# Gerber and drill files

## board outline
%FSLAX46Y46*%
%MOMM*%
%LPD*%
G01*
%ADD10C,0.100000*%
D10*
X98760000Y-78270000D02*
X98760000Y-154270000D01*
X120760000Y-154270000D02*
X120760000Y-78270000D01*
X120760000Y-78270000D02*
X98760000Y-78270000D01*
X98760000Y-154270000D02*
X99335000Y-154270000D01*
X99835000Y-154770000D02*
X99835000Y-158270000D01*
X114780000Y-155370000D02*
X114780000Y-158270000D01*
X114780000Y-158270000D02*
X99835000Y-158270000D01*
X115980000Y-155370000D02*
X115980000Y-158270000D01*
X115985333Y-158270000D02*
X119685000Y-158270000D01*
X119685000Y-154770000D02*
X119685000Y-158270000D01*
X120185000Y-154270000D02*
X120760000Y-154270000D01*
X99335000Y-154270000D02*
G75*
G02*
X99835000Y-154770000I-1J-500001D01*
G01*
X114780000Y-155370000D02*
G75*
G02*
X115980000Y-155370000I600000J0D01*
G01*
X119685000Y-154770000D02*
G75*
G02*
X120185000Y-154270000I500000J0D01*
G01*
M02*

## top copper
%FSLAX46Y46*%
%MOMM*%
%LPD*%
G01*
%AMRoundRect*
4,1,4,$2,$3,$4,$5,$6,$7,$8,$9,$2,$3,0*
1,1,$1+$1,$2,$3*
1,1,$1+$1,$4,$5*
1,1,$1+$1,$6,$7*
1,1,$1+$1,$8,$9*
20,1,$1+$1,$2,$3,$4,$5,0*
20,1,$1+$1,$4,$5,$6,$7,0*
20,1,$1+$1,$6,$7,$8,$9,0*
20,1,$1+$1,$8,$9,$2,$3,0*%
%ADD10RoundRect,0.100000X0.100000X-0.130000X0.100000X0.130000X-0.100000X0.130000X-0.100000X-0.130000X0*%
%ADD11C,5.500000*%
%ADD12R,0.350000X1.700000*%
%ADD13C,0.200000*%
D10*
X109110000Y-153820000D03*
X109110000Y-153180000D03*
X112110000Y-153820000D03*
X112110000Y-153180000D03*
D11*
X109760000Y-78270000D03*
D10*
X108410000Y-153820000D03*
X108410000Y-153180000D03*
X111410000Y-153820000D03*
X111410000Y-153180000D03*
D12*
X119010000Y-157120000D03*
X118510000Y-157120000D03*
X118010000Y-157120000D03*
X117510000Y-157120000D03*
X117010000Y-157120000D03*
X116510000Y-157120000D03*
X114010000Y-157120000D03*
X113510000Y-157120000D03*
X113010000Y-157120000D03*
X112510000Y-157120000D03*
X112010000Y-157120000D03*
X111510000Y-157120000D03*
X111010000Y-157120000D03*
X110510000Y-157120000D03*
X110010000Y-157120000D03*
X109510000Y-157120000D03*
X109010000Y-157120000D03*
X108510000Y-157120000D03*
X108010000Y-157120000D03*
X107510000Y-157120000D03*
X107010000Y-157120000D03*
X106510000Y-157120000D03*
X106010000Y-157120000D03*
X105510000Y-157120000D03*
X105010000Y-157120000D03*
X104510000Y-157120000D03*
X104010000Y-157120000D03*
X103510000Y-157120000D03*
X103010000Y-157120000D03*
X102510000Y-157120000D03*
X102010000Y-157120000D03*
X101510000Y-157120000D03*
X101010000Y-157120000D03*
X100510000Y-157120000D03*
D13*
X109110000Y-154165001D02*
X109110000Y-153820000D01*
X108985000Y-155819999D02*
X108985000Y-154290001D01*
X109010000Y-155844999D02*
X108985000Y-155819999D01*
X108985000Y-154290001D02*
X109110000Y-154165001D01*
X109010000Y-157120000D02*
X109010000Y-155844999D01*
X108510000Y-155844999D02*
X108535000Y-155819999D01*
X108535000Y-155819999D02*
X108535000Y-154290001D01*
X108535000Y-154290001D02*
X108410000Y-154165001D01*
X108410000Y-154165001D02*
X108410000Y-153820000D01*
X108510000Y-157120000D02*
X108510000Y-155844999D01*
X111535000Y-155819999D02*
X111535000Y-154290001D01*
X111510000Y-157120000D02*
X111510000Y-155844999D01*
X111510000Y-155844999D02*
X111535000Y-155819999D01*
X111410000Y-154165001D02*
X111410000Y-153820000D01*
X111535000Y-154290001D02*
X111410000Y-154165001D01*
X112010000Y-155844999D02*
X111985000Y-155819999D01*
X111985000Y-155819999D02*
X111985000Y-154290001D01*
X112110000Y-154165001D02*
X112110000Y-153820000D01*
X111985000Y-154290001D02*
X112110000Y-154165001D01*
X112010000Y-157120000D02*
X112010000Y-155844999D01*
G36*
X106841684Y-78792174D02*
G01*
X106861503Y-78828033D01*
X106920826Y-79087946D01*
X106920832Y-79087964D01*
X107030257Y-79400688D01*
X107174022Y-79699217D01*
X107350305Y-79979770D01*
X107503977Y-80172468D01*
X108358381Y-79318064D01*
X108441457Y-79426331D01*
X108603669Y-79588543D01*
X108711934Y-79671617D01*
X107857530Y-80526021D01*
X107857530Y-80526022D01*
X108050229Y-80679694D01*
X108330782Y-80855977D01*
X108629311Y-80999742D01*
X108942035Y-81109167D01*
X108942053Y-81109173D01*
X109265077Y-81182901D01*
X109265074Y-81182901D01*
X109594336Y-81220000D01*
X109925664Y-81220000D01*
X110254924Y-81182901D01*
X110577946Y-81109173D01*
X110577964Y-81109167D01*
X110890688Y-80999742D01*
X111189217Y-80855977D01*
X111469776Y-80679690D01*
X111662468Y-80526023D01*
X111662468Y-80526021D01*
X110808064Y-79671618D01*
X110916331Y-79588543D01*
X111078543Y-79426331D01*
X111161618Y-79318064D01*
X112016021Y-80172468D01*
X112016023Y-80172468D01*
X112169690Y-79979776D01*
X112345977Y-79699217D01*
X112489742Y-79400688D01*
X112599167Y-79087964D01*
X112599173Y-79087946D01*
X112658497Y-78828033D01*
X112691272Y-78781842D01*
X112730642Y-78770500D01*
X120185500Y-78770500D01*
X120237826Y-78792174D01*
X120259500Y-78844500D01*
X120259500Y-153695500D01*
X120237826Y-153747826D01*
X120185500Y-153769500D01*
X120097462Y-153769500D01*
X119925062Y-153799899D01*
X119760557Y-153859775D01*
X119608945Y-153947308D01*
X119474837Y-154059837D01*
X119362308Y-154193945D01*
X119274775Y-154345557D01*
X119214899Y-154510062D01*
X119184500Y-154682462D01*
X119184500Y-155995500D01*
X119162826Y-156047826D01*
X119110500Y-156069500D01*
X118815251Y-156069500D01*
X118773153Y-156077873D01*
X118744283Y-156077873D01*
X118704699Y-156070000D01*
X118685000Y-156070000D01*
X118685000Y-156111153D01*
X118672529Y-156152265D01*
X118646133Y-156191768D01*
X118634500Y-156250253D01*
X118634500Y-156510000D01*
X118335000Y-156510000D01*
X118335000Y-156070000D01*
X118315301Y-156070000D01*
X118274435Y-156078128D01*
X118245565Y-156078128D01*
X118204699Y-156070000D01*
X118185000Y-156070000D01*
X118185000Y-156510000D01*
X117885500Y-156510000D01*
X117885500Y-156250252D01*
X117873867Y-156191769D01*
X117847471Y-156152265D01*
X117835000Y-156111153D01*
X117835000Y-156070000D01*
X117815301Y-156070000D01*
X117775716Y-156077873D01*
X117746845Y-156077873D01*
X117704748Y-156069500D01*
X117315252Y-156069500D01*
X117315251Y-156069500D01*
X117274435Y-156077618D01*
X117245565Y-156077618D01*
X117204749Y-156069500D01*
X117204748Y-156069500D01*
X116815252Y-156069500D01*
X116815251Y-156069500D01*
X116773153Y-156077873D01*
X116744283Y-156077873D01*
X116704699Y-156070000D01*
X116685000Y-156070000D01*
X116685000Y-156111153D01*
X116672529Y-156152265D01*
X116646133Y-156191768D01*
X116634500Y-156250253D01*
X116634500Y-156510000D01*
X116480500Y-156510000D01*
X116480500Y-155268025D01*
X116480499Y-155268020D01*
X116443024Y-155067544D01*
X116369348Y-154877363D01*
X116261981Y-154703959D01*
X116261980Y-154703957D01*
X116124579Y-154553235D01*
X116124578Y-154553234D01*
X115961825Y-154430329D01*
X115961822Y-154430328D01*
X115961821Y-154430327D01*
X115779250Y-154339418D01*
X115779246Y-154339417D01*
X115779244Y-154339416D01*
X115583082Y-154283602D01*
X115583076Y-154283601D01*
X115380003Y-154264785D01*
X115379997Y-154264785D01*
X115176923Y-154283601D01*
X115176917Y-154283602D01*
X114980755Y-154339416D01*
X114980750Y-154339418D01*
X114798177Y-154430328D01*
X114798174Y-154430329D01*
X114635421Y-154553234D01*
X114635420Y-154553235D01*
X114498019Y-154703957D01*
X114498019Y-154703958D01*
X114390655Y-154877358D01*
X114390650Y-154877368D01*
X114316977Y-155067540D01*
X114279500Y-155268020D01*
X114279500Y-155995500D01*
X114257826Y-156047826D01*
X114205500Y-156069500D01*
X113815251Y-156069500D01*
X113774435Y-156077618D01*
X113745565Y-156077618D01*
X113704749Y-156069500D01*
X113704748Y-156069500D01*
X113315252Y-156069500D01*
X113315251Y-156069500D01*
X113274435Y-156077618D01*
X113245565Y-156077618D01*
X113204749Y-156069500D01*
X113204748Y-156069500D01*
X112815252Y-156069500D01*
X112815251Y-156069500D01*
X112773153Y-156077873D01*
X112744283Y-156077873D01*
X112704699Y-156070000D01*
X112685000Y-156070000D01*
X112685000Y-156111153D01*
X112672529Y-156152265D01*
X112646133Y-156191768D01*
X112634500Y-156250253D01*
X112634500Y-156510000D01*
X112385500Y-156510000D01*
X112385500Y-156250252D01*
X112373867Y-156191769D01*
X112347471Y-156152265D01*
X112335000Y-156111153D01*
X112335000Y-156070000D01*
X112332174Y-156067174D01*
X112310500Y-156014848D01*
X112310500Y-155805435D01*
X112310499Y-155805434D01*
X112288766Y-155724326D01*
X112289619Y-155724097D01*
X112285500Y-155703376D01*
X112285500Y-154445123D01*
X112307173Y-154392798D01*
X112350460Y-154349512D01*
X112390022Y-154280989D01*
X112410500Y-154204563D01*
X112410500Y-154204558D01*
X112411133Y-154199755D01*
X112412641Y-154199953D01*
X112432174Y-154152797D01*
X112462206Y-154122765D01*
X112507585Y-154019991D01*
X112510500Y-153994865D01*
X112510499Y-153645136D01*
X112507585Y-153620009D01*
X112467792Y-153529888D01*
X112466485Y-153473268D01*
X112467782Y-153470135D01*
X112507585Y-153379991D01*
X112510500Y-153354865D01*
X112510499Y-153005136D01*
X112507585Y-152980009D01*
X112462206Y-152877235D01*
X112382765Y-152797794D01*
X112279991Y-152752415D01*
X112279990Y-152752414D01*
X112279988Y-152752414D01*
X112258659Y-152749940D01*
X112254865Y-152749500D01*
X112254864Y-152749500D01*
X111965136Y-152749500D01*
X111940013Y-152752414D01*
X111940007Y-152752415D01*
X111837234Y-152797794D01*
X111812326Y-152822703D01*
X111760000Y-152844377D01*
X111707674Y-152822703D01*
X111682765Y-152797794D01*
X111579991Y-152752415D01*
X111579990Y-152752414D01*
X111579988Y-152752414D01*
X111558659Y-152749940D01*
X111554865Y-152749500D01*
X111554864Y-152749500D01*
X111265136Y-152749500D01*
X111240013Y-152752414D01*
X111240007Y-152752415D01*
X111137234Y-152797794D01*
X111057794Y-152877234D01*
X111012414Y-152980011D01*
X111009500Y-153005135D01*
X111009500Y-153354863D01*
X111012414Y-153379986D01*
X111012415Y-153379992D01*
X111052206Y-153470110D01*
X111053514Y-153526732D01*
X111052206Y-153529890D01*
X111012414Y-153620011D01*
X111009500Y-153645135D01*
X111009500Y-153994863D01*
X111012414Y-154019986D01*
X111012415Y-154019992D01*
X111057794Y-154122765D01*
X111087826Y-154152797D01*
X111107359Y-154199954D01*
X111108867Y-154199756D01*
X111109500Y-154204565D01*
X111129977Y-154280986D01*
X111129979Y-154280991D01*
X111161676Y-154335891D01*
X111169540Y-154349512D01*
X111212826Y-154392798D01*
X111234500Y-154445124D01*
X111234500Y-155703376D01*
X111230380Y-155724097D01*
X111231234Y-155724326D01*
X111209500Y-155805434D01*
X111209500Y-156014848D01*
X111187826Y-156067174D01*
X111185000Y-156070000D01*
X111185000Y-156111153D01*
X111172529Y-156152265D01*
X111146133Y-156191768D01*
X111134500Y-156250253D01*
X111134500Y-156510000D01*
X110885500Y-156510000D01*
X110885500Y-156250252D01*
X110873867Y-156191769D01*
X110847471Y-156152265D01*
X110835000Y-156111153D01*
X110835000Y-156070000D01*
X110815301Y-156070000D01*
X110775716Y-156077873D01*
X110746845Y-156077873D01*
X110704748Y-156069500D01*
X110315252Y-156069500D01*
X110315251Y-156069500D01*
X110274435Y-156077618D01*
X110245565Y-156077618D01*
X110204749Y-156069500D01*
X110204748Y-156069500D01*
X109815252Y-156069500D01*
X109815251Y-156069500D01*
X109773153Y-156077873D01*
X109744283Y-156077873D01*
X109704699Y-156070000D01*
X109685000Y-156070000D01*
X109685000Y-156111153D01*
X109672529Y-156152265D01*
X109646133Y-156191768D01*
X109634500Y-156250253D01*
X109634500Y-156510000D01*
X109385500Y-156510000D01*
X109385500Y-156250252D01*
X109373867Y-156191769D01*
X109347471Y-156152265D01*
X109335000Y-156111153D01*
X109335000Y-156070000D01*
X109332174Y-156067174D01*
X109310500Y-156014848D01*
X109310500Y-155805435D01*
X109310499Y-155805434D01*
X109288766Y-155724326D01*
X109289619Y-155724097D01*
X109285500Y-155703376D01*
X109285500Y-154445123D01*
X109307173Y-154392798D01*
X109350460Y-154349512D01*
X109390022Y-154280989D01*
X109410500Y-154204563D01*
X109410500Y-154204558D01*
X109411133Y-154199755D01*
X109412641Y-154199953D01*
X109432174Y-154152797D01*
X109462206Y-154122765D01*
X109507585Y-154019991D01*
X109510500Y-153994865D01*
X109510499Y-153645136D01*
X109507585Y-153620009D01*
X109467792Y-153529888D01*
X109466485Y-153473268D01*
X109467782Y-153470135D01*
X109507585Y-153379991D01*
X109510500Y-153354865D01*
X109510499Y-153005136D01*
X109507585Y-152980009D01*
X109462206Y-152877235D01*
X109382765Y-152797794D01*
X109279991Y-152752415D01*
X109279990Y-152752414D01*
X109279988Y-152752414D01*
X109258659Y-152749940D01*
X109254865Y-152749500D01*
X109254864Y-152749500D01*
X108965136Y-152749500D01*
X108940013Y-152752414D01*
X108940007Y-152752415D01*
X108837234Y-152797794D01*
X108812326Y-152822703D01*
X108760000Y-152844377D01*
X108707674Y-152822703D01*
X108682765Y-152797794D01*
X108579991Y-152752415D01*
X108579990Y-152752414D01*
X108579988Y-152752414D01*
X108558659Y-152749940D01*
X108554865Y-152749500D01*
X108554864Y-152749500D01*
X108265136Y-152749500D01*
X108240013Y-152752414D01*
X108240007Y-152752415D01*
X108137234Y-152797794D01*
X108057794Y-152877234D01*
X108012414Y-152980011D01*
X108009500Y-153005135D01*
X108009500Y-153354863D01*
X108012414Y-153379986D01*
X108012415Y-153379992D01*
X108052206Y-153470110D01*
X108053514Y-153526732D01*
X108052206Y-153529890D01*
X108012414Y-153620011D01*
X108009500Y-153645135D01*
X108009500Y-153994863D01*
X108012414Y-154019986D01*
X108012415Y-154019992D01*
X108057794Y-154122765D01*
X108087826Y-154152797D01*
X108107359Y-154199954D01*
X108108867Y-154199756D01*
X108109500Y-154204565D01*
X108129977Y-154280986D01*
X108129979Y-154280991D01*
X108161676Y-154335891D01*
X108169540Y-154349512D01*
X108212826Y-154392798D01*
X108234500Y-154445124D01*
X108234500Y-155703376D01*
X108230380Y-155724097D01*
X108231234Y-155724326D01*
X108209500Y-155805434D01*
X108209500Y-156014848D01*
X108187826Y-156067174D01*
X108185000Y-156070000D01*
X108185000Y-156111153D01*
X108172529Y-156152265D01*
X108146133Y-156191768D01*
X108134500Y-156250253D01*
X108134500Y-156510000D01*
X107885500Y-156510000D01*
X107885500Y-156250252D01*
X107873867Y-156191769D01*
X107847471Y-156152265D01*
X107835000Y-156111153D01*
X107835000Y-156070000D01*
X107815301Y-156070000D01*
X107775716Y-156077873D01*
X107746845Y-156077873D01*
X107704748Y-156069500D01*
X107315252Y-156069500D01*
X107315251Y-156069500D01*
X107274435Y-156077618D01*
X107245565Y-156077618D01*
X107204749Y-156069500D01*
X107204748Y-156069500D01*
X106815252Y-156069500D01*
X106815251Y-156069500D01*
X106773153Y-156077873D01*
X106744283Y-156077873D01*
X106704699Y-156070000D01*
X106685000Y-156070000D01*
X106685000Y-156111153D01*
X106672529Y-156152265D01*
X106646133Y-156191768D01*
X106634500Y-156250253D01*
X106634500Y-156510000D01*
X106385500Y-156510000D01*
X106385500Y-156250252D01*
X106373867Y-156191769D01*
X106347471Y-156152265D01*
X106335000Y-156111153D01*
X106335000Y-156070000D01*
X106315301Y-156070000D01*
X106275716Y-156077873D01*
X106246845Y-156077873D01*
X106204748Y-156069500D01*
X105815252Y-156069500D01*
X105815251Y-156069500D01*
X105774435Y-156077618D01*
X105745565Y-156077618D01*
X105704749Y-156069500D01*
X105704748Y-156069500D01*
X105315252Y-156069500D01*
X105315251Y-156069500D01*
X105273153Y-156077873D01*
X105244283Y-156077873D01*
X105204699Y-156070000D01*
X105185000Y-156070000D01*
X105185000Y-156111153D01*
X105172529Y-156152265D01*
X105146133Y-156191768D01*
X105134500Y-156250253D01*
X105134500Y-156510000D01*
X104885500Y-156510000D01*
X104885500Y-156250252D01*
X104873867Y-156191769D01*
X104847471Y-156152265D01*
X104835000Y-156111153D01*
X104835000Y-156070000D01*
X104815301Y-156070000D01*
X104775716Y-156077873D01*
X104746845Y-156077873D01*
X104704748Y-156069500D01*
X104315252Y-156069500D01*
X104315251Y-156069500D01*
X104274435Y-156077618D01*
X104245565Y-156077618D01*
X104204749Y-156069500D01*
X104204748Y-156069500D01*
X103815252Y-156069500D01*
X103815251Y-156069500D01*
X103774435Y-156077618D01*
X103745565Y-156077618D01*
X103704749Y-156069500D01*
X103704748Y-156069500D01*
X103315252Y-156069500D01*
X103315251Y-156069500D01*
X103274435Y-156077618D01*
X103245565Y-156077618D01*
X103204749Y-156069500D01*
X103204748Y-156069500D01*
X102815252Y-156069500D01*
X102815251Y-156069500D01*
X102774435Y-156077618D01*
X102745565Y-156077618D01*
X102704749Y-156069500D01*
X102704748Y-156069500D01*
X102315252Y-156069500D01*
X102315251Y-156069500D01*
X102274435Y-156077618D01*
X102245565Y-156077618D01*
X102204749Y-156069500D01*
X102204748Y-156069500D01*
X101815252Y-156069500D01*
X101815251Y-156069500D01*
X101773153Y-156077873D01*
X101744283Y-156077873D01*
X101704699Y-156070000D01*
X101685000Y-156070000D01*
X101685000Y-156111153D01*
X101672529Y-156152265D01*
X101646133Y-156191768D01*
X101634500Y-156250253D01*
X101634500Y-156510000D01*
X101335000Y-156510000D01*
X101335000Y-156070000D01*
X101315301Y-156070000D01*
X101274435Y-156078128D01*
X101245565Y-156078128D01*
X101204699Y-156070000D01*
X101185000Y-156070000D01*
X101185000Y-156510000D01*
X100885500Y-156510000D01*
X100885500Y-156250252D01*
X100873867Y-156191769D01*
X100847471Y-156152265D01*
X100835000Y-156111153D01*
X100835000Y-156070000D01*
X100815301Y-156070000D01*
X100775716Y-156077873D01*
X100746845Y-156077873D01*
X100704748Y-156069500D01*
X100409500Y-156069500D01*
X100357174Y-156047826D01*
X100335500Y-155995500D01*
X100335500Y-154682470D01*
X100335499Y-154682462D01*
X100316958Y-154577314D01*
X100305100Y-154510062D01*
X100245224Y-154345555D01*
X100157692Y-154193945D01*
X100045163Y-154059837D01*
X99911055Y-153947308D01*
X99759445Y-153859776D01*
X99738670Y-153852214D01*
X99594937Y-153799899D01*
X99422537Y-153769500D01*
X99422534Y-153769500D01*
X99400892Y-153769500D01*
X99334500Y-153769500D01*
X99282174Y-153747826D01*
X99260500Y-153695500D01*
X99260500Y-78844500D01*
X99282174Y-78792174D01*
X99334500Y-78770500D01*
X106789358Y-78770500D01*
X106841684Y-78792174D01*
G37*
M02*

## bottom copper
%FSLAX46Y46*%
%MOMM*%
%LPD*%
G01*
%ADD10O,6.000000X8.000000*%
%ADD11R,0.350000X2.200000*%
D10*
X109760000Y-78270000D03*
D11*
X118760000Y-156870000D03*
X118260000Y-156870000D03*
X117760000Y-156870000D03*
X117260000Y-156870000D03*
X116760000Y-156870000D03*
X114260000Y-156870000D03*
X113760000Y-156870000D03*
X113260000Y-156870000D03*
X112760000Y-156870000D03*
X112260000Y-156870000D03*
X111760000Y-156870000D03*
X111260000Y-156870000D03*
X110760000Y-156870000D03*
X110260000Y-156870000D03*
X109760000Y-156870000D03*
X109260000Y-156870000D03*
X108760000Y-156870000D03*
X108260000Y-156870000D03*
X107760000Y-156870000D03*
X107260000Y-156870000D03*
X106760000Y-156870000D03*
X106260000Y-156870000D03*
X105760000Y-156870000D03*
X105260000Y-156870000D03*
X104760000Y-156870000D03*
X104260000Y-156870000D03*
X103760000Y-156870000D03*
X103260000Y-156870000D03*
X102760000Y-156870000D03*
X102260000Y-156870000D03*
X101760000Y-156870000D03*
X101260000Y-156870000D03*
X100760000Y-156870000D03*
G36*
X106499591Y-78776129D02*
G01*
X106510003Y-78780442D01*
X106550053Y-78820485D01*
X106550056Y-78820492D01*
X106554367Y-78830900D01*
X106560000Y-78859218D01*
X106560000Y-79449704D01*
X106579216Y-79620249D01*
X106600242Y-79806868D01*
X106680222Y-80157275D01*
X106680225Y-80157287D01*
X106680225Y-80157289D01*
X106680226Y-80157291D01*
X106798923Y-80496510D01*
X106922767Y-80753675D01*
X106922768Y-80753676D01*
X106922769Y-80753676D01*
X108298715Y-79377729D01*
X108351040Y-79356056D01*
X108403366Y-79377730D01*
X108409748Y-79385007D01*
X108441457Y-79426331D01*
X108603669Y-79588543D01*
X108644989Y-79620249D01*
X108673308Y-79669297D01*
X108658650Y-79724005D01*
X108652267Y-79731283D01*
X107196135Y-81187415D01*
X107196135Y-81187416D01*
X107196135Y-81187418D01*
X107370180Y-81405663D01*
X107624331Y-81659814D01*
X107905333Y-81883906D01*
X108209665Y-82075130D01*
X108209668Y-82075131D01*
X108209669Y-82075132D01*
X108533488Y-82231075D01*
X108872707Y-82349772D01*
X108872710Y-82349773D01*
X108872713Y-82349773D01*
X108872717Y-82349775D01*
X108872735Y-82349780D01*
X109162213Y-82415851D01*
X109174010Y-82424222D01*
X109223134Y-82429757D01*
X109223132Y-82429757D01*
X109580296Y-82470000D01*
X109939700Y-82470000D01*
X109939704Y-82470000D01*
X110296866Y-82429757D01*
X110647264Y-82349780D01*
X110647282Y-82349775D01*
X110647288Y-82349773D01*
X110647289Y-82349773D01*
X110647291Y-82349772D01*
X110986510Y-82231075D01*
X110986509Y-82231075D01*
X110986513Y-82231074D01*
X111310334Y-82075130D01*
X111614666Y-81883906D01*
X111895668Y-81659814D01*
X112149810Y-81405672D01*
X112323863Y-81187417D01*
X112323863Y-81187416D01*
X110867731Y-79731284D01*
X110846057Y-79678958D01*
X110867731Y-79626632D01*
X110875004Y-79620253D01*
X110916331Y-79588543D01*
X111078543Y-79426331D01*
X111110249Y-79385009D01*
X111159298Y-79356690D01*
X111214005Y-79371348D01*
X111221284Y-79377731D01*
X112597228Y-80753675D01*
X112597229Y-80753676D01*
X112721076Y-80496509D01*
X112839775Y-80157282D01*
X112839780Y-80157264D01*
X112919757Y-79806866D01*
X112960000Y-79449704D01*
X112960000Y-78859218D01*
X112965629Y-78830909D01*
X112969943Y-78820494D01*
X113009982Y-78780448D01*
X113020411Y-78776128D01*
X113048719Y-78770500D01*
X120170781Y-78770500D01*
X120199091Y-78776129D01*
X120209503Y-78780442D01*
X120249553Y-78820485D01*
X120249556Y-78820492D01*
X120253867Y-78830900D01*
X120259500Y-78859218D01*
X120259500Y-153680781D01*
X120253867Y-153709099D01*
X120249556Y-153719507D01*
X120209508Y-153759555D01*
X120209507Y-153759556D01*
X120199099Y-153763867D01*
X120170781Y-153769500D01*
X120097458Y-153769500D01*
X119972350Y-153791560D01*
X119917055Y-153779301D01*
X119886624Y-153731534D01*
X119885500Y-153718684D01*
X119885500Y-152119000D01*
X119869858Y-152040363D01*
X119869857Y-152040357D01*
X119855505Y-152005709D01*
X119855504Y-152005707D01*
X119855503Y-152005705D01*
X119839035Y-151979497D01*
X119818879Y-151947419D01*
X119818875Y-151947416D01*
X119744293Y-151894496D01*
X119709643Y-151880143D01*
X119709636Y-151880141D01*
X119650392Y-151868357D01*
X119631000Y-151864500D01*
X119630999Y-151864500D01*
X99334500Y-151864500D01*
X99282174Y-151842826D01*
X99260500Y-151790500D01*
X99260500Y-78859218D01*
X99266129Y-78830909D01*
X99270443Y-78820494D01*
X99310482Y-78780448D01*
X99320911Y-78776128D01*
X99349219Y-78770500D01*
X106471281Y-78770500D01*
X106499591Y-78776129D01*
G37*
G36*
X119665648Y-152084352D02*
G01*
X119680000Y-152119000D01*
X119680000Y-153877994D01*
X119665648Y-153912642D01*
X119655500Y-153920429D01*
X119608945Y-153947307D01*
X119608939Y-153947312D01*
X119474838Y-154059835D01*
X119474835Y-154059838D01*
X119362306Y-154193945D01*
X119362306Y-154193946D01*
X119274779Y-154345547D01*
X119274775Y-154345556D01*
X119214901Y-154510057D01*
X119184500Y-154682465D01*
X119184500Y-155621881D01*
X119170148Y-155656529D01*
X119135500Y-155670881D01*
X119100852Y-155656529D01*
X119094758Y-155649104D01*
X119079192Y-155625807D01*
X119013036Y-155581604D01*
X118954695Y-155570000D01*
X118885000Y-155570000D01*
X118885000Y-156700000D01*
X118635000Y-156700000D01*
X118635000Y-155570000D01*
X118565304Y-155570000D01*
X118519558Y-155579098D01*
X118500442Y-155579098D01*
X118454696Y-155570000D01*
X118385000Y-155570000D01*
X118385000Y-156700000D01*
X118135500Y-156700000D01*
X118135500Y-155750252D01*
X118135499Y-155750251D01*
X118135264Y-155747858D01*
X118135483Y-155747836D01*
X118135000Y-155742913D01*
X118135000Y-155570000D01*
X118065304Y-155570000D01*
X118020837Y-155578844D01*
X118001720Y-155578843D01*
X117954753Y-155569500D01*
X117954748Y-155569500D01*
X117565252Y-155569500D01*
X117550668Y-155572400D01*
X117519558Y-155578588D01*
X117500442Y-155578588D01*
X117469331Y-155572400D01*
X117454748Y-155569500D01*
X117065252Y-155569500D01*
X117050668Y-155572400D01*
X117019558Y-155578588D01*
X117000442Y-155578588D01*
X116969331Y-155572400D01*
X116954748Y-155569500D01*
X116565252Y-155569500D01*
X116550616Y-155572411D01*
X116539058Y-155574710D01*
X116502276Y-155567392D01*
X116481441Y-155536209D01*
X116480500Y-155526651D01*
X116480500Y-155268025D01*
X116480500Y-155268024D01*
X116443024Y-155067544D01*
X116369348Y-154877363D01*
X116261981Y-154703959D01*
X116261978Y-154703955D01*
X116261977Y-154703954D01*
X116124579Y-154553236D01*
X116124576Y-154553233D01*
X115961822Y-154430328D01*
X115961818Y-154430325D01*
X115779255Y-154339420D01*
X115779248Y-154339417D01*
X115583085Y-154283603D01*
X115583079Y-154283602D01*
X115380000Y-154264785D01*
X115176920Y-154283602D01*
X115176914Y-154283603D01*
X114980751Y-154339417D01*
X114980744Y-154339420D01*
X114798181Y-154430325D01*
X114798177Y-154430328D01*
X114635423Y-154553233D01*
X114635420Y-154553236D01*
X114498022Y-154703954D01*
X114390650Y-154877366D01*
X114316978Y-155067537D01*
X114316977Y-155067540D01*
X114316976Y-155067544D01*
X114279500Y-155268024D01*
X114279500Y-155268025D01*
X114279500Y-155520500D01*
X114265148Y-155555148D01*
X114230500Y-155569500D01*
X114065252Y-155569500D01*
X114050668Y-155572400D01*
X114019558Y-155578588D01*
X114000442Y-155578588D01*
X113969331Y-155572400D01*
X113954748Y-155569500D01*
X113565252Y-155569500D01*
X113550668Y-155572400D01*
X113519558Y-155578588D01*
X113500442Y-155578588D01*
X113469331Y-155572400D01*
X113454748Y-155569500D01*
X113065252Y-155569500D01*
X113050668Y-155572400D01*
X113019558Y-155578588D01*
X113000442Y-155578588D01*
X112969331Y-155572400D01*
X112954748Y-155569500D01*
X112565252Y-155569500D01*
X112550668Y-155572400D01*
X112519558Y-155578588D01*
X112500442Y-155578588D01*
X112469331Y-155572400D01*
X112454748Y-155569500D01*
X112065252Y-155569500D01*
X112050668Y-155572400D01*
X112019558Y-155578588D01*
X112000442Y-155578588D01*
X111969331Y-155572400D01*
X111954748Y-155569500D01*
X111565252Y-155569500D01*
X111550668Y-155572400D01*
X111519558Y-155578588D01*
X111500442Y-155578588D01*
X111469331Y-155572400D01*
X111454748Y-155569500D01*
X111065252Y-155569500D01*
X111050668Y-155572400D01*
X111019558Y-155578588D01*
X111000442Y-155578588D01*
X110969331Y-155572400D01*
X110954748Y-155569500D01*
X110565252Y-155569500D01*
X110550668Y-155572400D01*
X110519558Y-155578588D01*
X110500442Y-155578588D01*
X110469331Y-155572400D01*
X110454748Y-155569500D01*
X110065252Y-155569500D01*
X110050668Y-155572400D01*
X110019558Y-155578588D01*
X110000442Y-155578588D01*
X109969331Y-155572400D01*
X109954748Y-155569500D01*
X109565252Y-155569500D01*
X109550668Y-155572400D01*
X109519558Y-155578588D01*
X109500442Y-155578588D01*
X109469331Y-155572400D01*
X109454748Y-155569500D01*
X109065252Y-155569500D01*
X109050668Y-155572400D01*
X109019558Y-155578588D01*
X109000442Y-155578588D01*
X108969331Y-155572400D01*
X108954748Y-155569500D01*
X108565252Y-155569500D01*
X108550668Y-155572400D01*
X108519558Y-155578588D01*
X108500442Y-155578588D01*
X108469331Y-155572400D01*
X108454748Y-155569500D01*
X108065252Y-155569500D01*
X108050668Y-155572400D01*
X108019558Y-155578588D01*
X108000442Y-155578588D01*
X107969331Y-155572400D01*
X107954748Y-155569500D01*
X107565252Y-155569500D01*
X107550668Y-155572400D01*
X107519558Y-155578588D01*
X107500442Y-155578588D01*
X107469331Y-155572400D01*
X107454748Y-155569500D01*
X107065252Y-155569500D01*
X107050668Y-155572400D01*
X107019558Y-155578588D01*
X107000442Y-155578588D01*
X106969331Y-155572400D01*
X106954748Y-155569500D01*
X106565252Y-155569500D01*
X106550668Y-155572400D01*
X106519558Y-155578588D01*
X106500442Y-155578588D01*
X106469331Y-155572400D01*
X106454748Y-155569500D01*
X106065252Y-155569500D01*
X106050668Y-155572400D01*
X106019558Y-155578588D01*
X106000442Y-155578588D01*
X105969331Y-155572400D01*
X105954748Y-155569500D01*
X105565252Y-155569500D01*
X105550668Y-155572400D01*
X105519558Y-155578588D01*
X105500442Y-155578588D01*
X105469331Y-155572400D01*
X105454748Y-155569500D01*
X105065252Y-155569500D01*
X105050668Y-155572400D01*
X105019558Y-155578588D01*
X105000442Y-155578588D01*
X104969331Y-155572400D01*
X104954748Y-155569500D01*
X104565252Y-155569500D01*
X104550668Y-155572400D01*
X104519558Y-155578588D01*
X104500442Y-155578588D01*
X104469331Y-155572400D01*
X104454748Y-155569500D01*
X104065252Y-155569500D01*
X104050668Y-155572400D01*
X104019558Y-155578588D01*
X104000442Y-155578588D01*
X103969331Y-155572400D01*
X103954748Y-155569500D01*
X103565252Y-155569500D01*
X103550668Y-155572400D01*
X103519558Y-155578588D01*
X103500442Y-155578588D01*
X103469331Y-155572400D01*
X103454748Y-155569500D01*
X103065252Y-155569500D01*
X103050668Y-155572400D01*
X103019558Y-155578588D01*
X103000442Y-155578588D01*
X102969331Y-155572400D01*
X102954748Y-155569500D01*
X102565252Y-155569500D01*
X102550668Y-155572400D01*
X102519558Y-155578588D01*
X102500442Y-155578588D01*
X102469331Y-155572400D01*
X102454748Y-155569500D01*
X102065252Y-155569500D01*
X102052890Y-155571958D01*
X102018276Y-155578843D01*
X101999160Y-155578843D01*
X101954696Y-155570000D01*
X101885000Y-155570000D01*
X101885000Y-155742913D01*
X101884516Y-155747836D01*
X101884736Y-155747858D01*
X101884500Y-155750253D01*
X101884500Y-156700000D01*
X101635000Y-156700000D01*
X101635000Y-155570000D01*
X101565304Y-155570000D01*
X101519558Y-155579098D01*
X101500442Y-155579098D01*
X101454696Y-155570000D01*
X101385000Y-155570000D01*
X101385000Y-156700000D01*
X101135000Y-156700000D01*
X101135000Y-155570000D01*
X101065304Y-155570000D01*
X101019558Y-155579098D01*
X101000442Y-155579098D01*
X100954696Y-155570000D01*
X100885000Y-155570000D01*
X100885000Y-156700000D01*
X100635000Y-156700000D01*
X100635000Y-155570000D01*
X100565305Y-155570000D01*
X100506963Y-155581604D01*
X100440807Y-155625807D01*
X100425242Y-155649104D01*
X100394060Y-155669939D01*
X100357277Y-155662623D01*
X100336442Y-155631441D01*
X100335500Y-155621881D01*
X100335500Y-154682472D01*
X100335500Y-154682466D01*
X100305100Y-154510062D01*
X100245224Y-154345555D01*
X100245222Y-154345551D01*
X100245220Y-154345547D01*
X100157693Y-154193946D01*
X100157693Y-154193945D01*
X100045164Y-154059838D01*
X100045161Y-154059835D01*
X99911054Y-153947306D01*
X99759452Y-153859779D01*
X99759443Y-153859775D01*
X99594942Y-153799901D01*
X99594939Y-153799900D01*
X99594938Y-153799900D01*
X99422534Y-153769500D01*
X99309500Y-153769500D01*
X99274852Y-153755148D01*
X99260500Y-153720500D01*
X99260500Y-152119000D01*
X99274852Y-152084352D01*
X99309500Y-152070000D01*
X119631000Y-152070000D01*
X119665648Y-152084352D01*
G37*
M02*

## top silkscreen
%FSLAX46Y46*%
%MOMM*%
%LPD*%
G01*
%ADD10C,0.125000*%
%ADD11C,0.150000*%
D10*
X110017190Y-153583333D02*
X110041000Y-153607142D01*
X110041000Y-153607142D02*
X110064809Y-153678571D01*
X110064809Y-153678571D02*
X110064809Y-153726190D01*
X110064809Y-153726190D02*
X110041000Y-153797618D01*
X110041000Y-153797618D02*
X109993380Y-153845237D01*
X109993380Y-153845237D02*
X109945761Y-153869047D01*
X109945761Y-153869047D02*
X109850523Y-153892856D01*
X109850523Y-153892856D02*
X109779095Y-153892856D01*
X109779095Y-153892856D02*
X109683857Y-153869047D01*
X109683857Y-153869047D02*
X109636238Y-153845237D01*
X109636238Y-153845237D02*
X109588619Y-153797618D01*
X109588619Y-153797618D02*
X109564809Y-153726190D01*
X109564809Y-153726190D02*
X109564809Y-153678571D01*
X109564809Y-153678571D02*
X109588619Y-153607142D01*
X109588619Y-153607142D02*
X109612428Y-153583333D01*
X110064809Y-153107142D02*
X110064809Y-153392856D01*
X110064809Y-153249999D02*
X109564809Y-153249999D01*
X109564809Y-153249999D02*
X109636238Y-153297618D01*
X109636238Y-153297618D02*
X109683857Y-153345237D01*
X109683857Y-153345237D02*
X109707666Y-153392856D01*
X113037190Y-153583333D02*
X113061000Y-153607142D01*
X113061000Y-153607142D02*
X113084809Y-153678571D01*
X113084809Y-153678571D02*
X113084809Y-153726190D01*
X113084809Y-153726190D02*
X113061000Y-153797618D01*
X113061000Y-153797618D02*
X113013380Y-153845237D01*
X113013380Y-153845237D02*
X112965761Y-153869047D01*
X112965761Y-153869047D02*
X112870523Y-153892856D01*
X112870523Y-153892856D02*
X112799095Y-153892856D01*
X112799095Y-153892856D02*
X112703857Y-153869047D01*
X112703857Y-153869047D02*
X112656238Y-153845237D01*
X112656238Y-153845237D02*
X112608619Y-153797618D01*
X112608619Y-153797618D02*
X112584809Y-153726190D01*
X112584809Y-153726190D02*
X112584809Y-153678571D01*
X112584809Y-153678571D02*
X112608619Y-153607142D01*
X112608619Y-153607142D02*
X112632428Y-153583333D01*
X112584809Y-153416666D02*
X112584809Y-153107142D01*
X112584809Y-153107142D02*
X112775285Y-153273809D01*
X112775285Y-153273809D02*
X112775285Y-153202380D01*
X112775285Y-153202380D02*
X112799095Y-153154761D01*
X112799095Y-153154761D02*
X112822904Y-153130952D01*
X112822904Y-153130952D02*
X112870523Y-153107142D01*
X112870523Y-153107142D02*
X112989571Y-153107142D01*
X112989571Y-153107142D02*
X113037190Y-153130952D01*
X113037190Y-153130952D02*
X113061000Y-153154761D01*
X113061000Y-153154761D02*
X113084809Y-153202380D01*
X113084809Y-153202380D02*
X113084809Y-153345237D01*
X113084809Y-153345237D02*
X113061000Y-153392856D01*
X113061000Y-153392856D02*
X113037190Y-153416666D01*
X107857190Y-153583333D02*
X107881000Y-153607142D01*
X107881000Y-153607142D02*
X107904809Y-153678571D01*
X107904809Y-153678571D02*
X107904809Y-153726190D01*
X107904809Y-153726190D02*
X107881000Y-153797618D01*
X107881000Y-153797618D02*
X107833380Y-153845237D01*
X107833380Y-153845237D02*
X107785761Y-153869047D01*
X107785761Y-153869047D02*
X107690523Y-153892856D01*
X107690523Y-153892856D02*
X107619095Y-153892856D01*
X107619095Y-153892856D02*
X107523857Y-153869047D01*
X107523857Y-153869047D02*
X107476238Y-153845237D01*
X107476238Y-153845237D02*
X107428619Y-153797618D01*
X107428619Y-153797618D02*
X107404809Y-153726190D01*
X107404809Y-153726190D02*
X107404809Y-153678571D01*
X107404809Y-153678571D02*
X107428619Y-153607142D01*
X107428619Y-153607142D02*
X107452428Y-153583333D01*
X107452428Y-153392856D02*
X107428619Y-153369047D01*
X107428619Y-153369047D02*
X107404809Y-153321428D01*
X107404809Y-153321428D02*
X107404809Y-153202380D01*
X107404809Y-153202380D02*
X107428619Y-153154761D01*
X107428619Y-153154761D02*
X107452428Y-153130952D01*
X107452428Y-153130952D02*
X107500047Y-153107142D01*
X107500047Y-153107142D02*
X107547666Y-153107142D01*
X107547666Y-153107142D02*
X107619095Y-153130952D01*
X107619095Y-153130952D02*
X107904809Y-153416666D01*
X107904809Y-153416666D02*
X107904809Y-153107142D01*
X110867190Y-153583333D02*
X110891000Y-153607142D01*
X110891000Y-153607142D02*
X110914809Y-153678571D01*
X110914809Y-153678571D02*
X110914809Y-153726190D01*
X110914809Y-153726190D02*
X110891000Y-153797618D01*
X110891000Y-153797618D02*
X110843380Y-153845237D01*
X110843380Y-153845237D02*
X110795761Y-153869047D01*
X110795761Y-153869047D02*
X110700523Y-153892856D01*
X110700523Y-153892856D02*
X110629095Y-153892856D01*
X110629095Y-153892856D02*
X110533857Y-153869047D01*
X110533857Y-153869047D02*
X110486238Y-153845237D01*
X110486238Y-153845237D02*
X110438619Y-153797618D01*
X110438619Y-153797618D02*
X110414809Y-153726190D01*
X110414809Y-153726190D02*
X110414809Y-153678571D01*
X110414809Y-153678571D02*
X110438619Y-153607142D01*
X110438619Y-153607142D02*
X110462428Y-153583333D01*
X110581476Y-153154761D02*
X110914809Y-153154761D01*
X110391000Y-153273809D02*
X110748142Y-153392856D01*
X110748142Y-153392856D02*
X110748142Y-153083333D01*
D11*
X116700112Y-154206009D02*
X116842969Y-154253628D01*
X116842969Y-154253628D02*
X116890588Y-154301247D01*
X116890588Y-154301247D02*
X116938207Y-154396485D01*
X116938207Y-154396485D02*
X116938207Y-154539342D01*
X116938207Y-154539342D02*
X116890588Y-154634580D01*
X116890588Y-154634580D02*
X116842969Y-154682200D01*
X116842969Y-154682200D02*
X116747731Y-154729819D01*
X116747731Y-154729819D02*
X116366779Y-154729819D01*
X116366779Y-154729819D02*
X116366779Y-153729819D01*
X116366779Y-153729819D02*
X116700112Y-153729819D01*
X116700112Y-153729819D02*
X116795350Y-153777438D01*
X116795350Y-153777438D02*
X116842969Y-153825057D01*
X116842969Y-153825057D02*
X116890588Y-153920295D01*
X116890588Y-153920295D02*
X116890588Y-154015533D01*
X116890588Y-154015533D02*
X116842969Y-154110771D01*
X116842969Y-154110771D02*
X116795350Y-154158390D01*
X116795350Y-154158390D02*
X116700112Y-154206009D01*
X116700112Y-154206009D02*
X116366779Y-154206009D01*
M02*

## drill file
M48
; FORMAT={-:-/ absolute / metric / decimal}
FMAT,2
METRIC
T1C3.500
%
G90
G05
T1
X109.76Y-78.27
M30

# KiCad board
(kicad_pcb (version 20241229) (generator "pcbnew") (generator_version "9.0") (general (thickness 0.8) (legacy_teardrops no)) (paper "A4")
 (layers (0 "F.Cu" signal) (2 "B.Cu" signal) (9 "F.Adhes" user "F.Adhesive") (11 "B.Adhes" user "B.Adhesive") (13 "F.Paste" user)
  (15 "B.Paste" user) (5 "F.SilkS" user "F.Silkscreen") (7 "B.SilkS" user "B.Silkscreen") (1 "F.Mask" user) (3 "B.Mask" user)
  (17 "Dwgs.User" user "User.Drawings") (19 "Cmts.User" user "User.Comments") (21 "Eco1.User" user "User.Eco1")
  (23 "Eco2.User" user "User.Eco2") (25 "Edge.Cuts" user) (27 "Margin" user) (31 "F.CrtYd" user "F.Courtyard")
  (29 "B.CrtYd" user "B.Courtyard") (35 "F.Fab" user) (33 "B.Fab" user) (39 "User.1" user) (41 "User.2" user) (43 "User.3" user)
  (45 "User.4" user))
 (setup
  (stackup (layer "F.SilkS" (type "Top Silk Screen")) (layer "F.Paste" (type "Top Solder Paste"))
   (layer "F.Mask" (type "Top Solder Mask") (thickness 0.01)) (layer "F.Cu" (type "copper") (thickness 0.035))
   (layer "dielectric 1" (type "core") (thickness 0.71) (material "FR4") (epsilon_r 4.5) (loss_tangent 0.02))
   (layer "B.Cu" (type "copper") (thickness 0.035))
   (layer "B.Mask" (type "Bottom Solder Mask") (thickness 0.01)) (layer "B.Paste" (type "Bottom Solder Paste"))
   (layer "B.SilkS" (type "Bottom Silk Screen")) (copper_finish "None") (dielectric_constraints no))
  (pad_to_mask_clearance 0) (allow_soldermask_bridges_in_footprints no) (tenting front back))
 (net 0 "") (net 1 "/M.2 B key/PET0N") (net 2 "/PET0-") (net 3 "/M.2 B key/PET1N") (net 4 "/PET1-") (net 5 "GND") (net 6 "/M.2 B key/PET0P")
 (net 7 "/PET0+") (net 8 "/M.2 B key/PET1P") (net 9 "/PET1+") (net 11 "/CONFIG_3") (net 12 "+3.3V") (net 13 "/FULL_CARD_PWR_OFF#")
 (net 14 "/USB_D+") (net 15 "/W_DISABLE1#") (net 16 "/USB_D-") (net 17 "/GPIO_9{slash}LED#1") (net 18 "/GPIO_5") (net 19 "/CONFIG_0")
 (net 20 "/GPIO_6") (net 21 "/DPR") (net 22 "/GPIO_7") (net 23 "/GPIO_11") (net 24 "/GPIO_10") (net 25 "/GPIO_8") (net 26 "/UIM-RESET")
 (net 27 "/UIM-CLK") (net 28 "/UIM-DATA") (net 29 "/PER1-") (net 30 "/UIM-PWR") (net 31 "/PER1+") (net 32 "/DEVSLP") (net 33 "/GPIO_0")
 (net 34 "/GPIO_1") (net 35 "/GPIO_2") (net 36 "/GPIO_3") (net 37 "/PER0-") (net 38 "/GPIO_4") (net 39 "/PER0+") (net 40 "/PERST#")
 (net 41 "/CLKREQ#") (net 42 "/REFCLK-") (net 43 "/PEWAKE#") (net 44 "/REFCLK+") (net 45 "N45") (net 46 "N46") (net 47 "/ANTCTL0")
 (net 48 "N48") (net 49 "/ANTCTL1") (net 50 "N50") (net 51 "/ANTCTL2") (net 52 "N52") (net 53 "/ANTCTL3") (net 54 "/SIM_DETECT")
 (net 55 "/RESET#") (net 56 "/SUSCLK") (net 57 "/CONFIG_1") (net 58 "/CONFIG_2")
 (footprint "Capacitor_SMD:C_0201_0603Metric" (layer "F.Cu") (at 109.11 153.5 90)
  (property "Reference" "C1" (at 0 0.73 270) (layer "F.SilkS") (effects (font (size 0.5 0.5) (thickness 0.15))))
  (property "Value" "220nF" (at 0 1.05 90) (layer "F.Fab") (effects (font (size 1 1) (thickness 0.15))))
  (pad "" smd roundrect (at -0.345 0 90) (size 0.318 0.36) (layers "F.Paste") (roundrect_rratio 0.25))
  (pad "" smd roundrect (at 0.345 0 90) (size 0.318 0.36) (layers "F.Paste") (roundrect_rratio 0.25))
  (pad "1" smd roundrect (at -0.32 0 90) (size 0.46 0.4) (layers "F.Cu" "F.Mask") (roundrect_rratio 0.25) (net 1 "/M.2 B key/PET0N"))
  (pad "2" smd roundrect (at 0.32 0 90) (size 0.46 0.4) (layers "F.Cu" "F.Mask") (roundrect_rratio 0.25) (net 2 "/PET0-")))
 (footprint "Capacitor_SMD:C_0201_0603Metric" (layer "F.Cu") (at 112.11 153.5 90)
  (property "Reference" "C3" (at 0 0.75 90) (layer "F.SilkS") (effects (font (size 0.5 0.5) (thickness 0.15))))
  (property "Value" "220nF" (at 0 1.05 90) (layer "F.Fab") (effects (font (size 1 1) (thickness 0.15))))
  (pad "" smd roundrect (at -0.345 0 90) (size 0.318 0.36) (layers "F.Paste") (roundrect_rratio 0.25))
  (pad "" smd roundrect (at 0.345 0 90) (size 0.318 0.36) (layers "F.Paste") (roundrect_rratio 0.25))
  (pad "1" smd roundrect (at -0.32 0 90) (size 0.46 0.4) (layers "F.Cu" "F.Mask") (roundrect_rratio 0.25) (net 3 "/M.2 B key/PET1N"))
  (pad "2" smd roundrect (at 0.32 0 90) (size 0.46 0.4) (layers "F.Cu" "F.Mask") (roundrect_rratio 0.25) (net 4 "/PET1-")))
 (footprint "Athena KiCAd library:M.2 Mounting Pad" (layer "F.Cu") (at 109.76 78.27)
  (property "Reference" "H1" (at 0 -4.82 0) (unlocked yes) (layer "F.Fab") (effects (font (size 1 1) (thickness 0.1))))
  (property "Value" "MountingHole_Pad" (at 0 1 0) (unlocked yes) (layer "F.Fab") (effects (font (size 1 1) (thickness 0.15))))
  (pad "1" thru_hole circle (at 0 0) (size 5.5 5.5) (drill 3.5) (layers "*.Cu" "*.Mask") (remove_unused_layers no) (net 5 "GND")
   (padstack (mode front_inner_back)
    (layer "Inner" (shape circle) (size 5.5 5.5) (zone_connect -1))
    (layer "B.Cu" (shape oval) (size 6 8) (thermal_bridge_angle 45) (zone_connect -1)))))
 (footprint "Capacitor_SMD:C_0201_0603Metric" (layer "F.Cu") (at 108.41 153.5 90)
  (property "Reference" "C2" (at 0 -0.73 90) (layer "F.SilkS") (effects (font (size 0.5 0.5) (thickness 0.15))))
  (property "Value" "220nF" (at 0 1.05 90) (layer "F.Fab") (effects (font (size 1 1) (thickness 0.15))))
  (pad "" smd roundrect (at -0.345 0 90) (size 0.318 0.36) (layers "F.Paste") (roundrect_rratio 0.25))
  (pad "" smd roundrect (at 0.345 0 90) (size 0.318 0.36) (layers "F.Paste") (roundrect_rratio 0.25))
  (pad "1" smd roundrect (at -0.32 0 90) (size 0.46 0.4) (layers "F.Cu" "F.Mask") (roundrect_rratio 0.25) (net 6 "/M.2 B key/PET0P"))
  (pad "2" smd roundrect (at 0.32 0 90) (size 0.46 0.4) (layers "F.Cu" "F.Mask") (roundrect_rratio 0.25) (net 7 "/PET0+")))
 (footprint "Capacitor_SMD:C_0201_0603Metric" (layer "F.Cu") (at 111.41 153.5 90)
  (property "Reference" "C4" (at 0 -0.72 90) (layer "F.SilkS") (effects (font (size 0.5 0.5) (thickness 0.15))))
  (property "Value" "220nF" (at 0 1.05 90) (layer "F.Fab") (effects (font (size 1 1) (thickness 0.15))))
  (pad "" smd roundrect (at -0.345 0 90) (size 0.318 0.36) (layers "F.Paste") (roundrect_rratio 0.25))
  (pad "" smd roundrect (at 0.345 0 90) (size 0.318 0.36) (layers "F.Paste") (roundrect_rratio 0.25))
  (pad "1" smd roundrect (at -0.32 0 90) (size 0.46 0.4) (layers "F.Cu" "F.Mask") (roundrect_rratio 0.25) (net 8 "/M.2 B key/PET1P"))
  (pad "2" smd roundrect (at 0.32 0 90) (size 0.46 0.4) (layers "F.Cu" "F.Mask") (roundrect_rratio 0.25) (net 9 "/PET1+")))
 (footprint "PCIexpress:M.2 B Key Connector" (layer "F.Cu") (at 109.76 157.16)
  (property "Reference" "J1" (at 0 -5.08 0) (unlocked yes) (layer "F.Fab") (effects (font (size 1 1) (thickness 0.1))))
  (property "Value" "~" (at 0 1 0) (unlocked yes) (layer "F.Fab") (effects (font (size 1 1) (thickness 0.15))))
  (fp_line (start -11 -2.89) (end -10.425 -2.89) (stroke (width 0.1) (type default)) (layer "Edge.Cuts") (net 10))
  (fp_line (start -9.925 -2.39) (end -9.925 1.11) (stroke (width 0.1) (type default)) (layer "Edge.Cuts") (net 10))
  (fp_line (start 5.02 -1.79) (end 5.02 1.11) (stroke (width 0.1) (type default)) (layer "Edge.Cuts") (net 10))
  (fp_line (start 5.02 1.11) (end -9.925 1.11) (stroke (width 0.1) (type default)) (layer "Edge.Cuts") (net 10))
  (fp_line (start 6.22 -1.79) (end 6.22 1.11) (stroke (width 0.1) (type default)) (layer "Edge.Cuts") (net 10))
  (fp_line (start 6.225333 1.11) (end 9.925 1.11) (stroke (width 0.1) (type default)) (layer "Edge.Cuts") (net 10))
  (fp_line (start 9.925 -2.39) (end 9.925 1.11) (stroke (width 0.1) (type default)) (layer "Edge.Cuts") (net 10))
  (fp_line (start 10.425 -2.89) (end 11 -2.89) (stroke (width 0.1) (type default)) (layer "Edge.Cuts") (net 10))
  (fp_arc (start -10.425 -2.89) (mid -10.071447 -2.743553) (end -9.925 -2.39) (stroke (width 0.1) (type default)) (layer "Edge.Cuts")
   (net 10))
  (fp_arc (start 5.02 -1.79) (mid 5.62 -2.39) (end 6.22 -1.79) (stroke (width 0.1) (type default)) (layer "Edge.Cuts") (net 10))
  (fp_arc (start 9.925 -2.39) (mid 10.071447 -2.743553) (end 10.425 -2.89) (stroke (width 0.1) (type default)) (layer "Edge.Cuts") (net 10))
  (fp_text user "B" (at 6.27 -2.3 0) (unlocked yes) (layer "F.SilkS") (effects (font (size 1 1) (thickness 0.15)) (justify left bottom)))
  (pad "1" smd rect (at 9.25 -0.04 180) (size 0.35 1.7) (layers "F.Cu") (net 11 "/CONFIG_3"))
  (pad "2" smd rect (at 9 -0.29 180) (size 0.35 2.2) (layers "B.Cu") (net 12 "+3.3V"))
  (pad "3" smd rect (at 8.75 -0.04 180) (size 0.35 1.7) (layers "F.Cu") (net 5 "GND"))
  (pad "4" smd rect (at 8.5 -0.29 180) (size 0.35 2.2) (layers "B.Cu") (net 12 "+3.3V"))
  (pad "5" smd rect (at 8.25 -0.04 180) (size 0.35 1.7) (layers "F.Cu") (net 5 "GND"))
  (pad "6" smd rect (at 8 -0.29 180) (size 0.35 2.2) (layers "B.Cu") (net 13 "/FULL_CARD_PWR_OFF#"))
  (pad "7" smd rect (at 7.75 -0.04 180) (size 0.35 1.7) (layers "F.Cu") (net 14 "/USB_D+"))
  (pad "8" smd rect (at 7.5 -0.29 180) (size 0.35 2.2) (layers "B.Cu") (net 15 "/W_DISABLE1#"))
  (pad "9" smd rect (at 7.25 -0.04 180) (size 0.35 1.7) (layers "F.Cu") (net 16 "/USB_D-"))
  (pad "10" smd rect (at 7 -0.29 180) (size 0.35 2.2) (layers "B.Cu") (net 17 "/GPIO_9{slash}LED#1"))
  (pad "11" smd rect (at 6.75 -0.04 180) (size 0.35 1.7) (layers "F.Cu") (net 5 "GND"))
  (pad "20" smd rect (at 4.5 -0.29 180) (size 0.35 2.2) (layers "B.Cu") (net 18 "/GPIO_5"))
  (pad "21" smd rect (at 4.25 -0.04 180) (size 0.35 1.7) (layers "F.Cu") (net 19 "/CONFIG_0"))
  (pad "22" smd rect (at 4 -0.29 180) (size 0.35 2.2) (layers "B.Cu") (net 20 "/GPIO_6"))
  (pad "23" smd rect (at 3.75 -0.04 180) (size 0.35 1.7) (layers "F.Cu") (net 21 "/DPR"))
  (pad "24" smd rect (at 3.5 -0.29 180) (size 0.35 2.2) (layers "B.Cu") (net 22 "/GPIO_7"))
  (pad "25" smd rect (at 3.25 -0.04 180) (size 0.35 1.7) (layers "F.Cu") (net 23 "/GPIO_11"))
  (pad "26" smd rect (at 3 -0.29 180) (size 0.35 2.2) (layers "B.Cu") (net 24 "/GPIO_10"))
  (pad "27" smd rect (at 2.75 -0.04 180) (size 0.35 1.7) (layers "F.Cu") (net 5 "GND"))
  (pad "28" smd rect (at 2.5 -0.29 180) (size 0.35 2.2) (layers "B.Cu") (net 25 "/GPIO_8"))
  (pad "29" smd rect (at 2.25 -0.04 180) (size 0.35 1.7) (layers "F.Cu") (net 3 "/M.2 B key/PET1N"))
  (pad "30" smd rect (at 2 -0.29 180) (size 0.35 2.2) (layers "B.Cu") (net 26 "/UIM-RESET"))
  (pad "31" smd rect (at 1.75 -0.04 180) (size 0.35 1.7) (layers "F.Cu") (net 8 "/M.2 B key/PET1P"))
  (pad "32" smd rect (at 1.5 -0.29 180) (size 0.35 2.2) (layers "B.Cu") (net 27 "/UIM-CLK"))
  (pad "33" smd rect (at 1.25 -0.04 180) (size 0.35 1.7) (layers "F.Cu") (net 5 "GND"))
  (pad "34" smd rect (at 1 -0.29 180) (size 0.35 2.2) (layers "B.Cu") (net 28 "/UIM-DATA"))
  (pad "35" smd rect (at 0.75 -0.04 180) (size 0.35 1.7) (layers "F.Cu") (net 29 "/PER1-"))
  (pad "36" smd rect (at 0.5 -0.29 180) (size 0.35 2.2) (layers "B.Cu") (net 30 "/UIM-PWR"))
  (pad "37" smd rect (at 0.25 -0.04 180) (size 0.35 1.7) (layers "F.Cu") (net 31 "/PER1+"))
  (pad "38" smd rect (at 0 -0.29 180) (size 0.35 2.2) (layers "B.Cu") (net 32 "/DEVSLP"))
  (pad "39" smd rect (at -0.25 -0.04 180) (size 0.35 1.7) (layers "F.Cu") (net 5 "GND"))
  (pad "40" smd rect (at -0.5 -0.29 180) (size 0.35 2.2) (layers "B.Cu") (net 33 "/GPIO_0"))
  (pad "41" smd rect (at -0.75 -0.04 180) (size 0.35 1.7) (layers "F.Cu") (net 1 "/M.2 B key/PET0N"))
  (pad "42" smd rect (at -1 -0.29 180) (size 0.35 2.2) (layers "B.Cu") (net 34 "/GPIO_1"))
  (pad "43" smd rect (at -1.25 -0.04 180) (size 0.35 1.7) (layers "F.Cu") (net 6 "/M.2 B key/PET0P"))
  (pad "44" smd rect (at -1.5 -0.29 180) (size 0.35 2.2) (layers "B.Cu") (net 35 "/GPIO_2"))
  (pad "45" smd rect (at -1.75 -0.04 180) (size 0.35 1.7) (layers "F.Cu") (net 5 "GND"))
  (pad "46" smd rect (at -2 -0.29 180) (size 0.35 2.2) (layers "B.Cu") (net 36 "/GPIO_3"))
  (pad "47" smd rect (at -2.25 -0.04 180) (size 0.35 1.7) (layers "F.Cu") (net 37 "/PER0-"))
  (pad "48" smd rect (at -2.5 -0.29 180) (size 0.35 2.2) (layers "B.Cu") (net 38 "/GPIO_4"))
  (pad "49" smd rect (at -2.75 -0.04 180) (size 0.35 1.7) (layers "F.Cu") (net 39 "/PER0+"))
  (pad "50" smd rect (at -3 -0.29 180) (size 0.35 2.2) (layers "B.Cu") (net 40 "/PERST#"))
  (pad "51" smd rect (at -3.25 -0.04 180) (size 0.35 1.7) (layers "F.Cu") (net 5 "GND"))
  (pad "52" smd rect (at -3.5 -0.29 180) (size 0.35 2.2) (layers "B.Cu") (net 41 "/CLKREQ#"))
  (pad "53" smd rect (at -3.75 -0.04 180) (size 0.35 1.7) (layers "F.Cu") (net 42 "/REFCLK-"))
  (pad "54" smd rect (at -4 -0.29 180) (size 0.35 2.2) (layers "B.Cu") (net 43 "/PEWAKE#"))
  (pad "55" smd rect (at -4.25 -0.04 180) (size 0.35 1.7) (layers "F.Cu") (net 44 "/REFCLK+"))
  (pad "56" smd rect (at -4.5 -0.29 180) (size 0.35 2.2) (layers "B.Cu") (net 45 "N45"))
  (pad "57" smd rect (at -4.75 -0.04 180) (size 0.35 1.7) (layers "F.Cu") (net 5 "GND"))
  (pad "58" smd rect (at -5 -0.29 180) (size 0.35 2.2) (layers "B.Cu") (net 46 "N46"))
  (pad "59" smd rect (at -5.25 -0.04 180) (size 0.35 1.7) (layers "F.Cu") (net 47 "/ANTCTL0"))
  (pad "60" smd rect (at -5.5 -0.29 180) (size 0.35 2.2) (layers "B.Cu") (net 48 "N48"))
  (pad "61" smd rect (at -5.75 -0.04 180) (size 0.35 1.7) (layers "F.Cu") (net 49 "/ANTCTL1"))
  (pad "62" smd rect (at -6 -0.29 180) (size 0.35 2.2) (layers "B.Cu") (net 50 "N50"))
  (pad "63" smd rect (at -6.25 -0.04 180) (size 0.35 1.7) (layers "F.Cu") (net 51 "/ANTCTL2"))
  (pad "64" smd rect (at -6.5 -0.29 180) (size 0.35 2.2) (layers "B.Cu") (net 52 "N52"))
  (pad "65" smd rect (at -6.75 -0.04 180) (size 0.35 1.7) (layers "F.Cu") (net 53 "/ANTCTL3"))
  (pad "66" smd rect (at -7 -0.29 180) (size 0.35 2.2) (layers "B.Cu") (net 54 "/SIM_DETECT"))
  (pad "67" smd rect (at -7.25 -0.04 180) (size 0.35 1.7) (layers "F.Cu") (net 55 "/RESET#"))
  (pad "68" smd rect (at -7.5 -0.29 180) (size 0.35 2.2) (layers "B.Cu") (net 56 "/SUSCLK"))
  (pad "69" smd rect (at -7.75 -0.04 180) (size 0.35 1.7) (layers "F.Cu") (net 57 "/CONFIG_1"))
  (pad "70" smd rect (at -8 -0.29 180) (size 0.35 2.2) (layers "B.Cu") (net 12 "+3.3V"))
  (pad "71" smd rect (at -8.25 -0.04 180) (size 0.35 1.7) (layers "F.Cu") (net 5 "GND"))
  (pad "72" smd rect (at -8.5 -0.29 180) (size 0.35 2.2) (layers "B.Cu") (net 12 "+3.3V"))
  (pad "73" smd rect (at -8.75 -0.04 180) (size 0.35 1.7) (layers "F.Cu") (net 5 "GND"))
  (pad "74" smd rect (at -9 -0.29 180) (size 0.35 2.2) (layers "B.Cu") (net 12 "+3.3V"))
  (pad "75" smd rect (at -9.25 -0.04 180) (size 0.35 1.7) (layers "F.Cu") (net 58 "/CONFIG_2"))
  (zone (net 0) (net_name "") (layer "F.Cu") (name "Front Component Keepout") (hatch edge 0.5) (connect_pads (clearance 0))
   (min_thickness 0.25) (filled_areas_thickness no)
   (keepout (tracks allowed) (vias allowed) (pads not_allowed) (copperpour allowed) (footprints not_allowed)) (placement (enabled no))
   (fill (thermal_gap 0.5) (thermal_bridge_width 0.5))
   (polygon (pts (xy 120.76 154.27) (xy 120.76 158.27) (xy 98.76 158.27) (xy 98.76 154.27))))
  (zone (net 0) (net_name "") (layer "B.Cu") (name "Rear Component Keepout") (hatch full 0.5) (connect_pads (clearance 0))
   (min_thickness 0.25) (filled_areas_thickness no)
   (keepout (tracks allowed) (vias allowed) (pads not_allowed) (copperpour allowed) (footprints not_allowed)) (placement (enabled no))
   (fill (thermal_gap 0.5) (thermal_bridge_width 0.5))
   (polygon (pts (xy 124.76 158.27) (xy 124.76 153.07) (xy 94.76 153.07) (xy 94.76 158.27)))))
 (gr_line (start 98.76 78.27) (end 98.76 154.27) (stroke (width 0.1) (type default)) (layer "Edge.Cuts"))
 (gr_line (start 120.76 154.27) (end 120.76 78.27) (stroke (width 0.1) (type default)) (layer "Edge.Cuts"))
 (gr_line (start 120.76 78.27) (end 98.76 78.27) (stroke (width 0.1) (type default)) (layer "Edge.Cuts"))
 (segment (start 109.11 154.165001) (end 109.11 153.82) (width 0.2) (layer "F.Cu") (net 1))
 (segment (start 108.985 155.819999) (end 108.985 154.290001) (width 0.2) (layer "F.Cu") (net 1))
 (segment (start 109.01 155.844999) (end 108.985 155.819999) (width 0.2) (layer "F.Cu") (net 1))
 (segment (start 108.985 154.290001) (end 109.11 154.165001) (width 0.2) (layer "F.Cu") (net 1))
 (segment (start 109.01 157.12) (end 109.01 155.844999) (width 0.2) (layer "F.Cu") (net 1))
 (segment (start 108.51 155.844999) (end 108.535 155.819999) (width 0.2) (layer "F.Cu") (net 6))
 (segment (start 108.535 155.819999) (end 108.535 154.290001) (width 0.2) (layer "F.Cu") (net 6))
 (segment (start 108.535 154.290001) (end 108.41 154.165001) (width 0.2) (layer "F.Cu") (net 6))
 (segment (start 108.41 154.165001) (end 108.41 153.82) (width 0.2) (layer "F.Cu") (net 6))
 (segment (start 108.51 157.12) (end 108.51 155.844999) (width 0.2) (layer "F.Cu") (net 6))
 (segment (start 111.535 155.819999) (end 111.535 154.290001) (width 0.2) (layer "F.Cu") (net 8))
 (segment (start 111.51 157.12) (end 111.51 155.844999) (width 0.2) (layer "F.Cu") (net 8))
 (segment (start 111.51 155.844999) (end 111.535 155.819999) (width 0.2) (layer "F.Cu") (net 8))
 (segment (start 111.41 154.165001) (end 111.41 153.82) (width 0.2) (layer "F.Cu") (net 8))
 (segment (start 111.535 154.290001) (end 111.41 154.165001) (width 0.2) (layer "F.Cu") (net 8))
 (segment (start 112.01 155.844999) (end 111.985 155.819999) (width 0.2) (layer "F.Cu") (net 3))
 (segment (start 111.985 155.819999) (end 111.985 154.290001) (width 0.2) (layer "F.Cu") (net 3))
 (segment (start 112.11 154.165001) (end 112.11 153.82) (width 0.2) (layer "F.Cu") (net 3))
 (segment (start 111.985 154.290001) (end 112.11 154.165001) (width 0.2) (layer "F.Cu") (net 3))
 (segment (start 112.01 157.12) (end 112.01 155.844999) (width 0.2) (layer "F.Cu") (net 3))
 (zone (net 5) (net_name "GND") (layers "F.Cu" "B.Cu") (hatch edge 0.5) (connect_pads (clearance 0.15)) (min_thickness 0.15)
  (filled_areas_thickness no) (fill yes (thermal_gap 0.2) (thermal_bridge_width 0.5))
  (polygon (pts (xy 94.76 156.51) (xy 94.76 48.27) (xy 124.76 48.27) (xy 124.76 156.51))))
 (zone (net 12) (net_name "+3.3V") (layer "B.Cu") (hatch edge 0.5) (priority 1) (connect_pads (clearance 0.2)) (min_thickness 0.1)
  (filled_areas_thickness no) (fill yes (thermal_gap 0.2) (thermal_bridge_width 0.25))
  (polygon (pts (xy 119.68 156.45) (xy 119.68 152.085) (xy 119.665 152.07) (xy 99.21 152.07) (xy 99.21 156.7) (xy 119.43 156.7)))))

